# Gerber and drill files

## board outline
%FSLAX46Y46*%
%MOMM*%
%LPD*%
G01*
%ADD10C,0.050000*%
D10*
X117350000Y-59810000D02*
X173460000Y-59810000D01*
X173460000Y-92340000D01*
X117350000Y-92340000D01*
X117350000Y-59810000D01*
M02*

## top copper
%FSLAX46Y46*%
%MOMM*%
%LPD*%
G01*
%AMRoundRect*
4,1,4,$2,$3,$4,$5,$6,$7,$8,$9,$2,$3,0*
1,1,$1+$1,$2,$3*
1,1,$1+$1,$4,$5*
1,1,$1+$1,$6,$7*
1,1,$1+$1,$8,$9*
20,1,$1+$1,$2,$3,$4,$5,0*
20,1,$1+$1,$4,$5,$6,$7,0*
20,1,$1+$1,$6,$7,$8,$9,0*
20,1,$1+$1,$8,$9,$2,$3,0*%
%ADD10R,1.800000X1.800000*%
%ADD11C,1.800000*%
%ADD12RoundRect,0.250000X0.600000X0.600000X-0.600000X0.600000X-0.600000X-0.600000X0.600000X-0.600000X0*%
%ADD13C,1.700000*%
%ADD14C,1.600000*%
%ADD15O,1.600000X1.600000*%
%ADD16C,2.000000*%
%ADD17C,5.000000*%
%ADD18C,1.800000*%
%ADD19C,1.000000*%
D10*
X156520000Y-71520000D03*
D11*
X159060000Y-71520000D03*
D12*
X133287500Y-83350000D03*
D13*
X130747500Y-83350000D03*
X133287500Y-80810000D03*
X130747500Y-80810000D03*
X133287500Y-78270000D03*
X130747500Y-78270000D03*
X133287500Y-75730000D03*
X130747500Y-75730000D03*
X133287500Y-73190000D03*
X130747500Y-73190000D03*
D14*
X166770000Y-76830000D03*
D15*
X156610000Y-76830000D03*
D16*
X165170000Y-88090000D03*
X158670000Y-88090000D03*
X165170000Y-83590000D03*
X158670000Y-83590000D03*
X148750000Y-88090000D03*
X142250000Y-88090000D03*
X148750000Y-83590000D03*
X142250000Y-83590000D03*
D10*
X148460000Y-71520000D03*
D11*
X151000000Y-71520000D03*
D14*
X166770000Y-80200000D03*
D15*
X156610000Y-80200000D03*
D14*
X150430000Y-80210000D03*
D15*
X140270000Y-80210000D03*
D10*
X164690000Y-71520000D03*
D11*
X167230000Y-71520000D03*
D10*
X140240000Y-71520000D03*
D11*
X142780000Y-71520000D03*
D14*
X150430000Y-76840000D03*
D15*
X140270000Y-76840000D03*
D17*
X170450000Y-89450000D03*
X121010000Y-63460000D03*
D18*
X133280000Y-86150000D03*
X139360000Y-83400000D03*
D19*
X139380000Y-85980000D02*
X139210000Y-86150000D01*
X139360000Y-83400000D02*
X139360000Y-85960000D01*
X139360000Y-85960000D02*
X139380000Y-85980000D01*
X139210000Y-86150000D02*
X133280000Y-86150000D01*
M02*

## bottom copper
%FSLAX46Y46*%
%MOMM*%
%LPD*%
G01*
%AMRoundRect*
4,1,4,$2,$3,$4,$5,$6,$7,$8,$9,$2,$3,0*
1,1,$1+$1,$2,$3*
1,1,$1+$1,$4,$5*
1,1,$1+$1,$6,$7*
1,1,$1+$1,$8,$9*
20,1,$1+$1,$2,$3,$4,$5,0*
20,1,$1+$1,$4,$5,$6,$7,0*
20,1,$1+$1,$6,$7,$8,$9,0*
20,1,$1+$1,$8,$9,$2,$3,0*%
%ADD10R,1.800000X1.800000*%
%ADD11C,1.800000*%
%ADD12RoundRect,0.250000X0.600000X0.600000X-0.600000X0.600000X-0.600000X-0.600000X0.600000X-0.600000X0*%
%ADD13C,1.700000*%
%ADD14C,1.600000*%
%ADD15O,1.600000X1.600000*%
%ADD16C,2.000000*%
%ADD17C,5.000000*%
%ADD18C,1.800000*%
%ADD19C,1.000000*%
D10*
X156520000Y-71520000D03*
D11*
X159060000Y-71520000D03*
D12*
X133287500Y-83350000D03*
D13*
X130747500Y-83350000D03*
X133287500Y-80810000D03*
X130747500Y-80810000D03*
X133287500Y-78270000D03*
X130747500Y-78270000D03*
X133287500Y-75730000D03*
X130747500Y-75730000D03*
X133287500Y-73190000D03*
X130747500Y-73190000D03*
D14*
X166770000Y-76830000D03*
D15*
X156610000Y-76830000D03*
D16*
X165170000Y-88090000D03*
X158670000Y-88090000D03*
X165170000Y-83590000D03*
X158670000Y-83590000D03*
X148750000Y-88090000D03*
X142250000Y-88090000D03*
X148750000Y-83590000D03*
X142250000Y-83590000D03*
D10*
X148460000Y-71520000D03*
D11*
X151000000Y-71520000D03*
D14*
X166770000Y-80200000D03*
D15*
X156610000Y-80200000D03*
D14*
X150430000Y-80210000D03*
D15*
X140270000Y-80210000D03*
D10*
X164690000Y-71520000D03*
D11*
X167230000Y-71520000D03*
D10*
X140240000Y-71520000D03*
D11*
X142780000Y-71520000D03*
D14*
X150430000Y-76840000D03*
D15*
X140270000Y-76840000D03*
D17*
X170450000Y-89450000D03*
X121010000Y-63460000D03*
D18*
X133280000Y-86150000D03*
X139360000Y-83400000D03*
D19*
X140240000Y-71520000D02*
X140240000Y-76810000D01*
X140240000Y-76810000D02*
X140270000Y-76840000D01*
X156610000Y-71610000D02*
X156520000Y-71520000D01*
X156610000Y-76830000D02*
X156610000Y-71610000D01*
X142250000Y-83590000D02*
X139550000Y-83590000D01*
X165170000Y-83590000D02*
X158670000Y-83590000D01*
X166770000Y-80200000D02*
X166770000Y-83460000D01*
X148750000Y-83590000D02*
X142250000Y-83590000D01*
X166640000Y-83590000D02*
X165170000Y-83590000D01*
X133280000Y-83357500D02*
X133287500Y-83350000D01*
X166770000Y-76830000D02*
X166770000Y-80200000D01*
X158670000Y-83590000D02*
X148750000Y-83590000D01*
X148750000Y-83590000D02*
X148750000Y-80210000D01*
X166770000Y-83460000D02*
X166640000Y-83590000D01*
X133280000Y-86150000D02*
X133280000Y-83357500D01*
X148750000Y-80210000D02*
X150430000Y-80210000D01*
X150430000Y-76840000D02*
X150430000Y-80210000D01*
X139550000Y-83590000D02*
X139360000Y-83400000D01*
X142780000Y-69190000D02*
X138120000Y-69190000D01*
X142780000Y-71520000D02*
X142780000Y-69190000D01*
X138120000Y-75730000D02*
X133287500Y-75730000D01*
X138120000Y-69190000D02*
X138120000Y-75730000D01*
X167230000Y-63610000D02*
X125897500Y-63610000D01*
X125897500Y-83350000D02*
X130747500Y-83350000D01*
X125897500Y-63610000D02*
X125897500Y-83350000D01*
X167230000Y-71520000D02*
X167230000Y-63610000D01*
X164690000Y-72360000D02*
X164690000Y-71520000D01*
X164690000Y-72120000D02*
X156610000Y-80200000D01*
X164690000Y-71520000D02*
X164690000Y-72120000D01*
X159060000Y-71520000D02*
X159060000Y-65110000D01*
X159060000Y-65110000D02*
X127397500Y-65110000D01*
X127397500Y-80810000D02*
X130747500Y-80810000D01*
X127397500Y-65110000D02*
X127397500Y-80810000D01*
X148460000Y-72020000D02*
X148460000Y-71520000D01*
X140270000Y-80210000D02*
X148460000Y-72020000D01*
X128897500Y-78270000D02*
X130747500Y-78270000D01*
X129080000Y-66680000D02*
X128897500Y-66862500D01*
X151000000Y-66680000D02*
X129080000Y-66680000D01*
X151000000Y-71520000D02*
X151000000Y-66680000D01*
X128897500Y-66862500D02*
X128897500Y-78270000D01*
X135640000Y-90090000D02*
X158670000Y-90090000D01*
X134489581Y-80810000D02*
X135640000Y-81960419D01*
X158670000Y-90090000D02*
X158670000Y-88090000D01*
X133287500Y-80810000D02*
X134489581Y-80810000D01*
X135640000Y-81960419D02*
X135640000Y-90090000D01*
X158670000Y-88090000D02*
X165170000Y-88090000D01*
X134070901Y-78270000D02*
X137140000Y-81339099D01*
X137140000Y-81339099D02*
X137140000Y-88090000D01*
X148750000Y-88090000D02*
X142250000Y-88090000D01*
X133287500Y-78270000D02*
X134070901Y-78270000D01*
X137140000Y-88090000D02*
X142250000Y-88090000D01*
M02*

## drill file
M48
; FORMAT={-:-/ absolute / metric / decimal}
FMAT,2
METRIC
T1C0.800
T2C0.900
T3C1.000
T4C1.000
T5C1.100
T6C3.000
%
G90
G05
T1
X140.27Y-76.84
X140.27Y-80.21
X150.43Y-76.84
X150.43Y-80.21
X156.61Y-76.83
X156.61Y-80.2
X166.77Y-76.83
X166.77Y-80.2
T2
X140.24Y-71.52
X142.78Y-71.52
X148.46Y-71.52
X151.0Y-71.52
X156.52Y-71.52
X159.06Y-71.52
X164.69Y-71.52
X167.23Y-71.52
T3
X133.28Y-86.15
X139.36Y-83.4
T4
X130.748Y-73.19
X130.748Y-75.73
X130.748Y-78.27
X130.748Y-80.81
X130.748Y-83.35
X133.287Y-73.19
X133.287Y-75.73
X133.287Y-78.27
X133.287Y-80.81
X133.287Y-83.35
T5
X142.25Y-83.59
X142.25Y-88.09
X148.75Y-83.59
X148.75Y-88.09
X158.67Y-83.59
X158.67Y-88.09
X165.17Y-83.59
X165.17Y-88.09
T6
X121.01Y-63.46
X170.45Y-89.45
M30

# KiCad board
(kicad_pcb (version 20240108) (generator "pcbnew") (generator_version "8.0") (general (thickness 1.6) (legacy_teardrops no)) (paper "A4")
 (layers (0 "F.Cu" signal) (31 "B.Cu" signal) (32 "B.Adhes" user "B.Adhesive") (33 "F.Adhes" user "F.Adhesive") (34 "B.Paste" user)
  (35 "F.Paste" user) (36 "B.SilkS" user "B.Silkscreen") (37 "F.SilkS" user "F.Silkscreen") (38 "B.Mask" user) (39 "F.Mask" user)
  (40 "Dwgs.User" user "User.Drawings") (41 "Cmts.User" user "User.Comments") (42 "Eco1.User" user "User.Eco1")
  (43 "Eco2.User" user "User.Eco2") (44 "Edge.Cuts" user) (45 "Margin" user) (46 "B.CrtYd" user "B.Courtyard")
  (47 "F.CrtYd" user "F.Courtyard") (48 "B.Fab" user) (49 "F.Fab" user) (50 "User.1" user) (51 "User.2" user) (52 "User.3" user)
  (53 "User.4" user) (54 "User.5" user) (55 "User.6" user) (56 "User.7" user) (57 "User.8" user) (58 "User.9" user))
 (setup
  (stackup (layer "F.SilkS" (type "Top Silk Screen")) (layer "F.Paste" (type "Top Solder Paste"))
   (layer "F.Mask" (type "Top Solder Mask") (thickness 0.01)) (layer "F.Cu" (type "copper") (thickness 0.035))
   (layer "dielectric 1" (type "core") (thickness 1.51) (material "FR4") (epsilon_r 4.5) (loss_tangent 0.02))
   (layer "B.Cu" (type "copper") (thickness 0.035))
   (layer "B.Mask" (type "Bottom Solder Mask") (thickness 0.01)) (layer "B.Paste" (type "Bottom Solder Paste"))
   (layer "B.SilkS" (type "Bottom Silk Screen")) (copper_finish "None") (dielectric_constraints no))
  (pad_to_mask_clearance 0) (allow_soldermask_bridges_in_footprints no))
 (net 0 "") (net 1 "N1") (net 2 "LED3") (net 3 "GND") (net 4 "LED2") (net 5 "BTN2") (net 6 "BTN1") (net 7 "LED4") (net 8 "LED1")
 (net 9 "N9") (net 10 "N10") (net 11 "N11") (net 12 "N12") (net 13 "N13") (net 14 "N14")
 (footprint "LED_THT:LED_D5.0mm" (layer "F.Cu") (at 156.52 71.52)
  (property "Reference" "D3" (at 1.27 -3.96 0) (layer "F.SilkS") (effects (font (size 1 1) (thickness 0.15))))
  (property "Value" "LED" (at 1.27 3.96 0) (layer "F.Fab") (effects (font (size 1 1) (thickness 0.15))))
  (pad "1" thru_hole rect (at 0 0) (size 1.8 1.8) (drill 0.9) (layers "*.Cu" "*.Mask") (remove_unused_layers no) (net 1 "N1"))
  (pad "2" thru_hole circle (at 2.54 0) (size 1.8 1.8) (drill 0.9) (layers "*.Cu" "*.Mask") (remove_unused_layers no) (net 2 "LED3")))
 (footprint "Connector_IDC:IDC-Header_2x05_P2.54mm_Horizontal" (layer "F.Cu") (at 133.2875 83.35 180)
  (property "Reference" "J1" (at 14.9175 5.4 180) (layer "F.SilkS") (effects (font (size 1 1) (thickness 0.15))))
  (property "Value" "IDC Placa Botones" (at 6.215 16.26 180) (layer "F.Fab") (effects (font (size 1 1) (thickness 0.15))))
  (pad "1" thru_hole roundrect (at 0 0 180) (size 1.7 1.7) (drill 1) (layers "*.Cu" "*.Mask") (remove_unused_layers no)
   (roundrect_rratio 0.147059) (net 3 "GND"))
  (pad "2" thru_hole circle (at 2.54 0 180) (size 1.7 1.7) (drill 1) (layers "*.Cu" "*.Mask") (remove_unused_layers no) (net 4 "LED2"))
  (pad "3" thru_hole circle (at 0 2.54 180) (size 1.7 1.7) (drill 1) (layers "*.Cu" "*.Mask") (remove_unused_layers no) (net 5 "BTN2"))
  (pad "4" thru_hole circle (at 2.54 2.54 180) (size 1.7 1.7) (drill 1) (layers "*.Cu" "*.Mask") (remove_unused_layers no) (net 2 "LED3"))
  (pad "5" thru_hole circle (at 0 5.08 180) (size 1.7 1.7) (drill 1) (layers "*.Cu" "*.Mask") (remove_unused_layers no) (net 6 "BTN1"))
  (pad "6" thru_hole circle (at 2.54 5.08 180) (size 1.7 1.7) (drill 1) (layers "*.Cu" "*.Mask") (remove_unused_layers no) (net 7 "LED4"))
  (pad "7" thru_hole circle (at 0 7.62 180) (size 1.7 1.7) (drill 1) (layers "*.Cu" "*.Mask") (remove_unused_layers no) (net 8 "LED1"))
  (pad "8" thru_hole circle (at 2.54 7.62 180) (size 1.7 1.7) (drill 1) (layers "*.Cu" "*.Mask") (remove_unused_layers no) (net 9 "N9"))
  (pad "9" thru_hole circle (at 0 10.16 180) (size 1.7 1.7) (drill 1) (layers "*.Cu" "*.Mask") (remove_unused_layers no) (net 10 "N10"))
  (pad "10" thru_hole circle (at 2.54 10.16 180) (size 1.7 1.7) (drill 1) (layers "*.Cu" "*.Mask") (remove_unused_layers no) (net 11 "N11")))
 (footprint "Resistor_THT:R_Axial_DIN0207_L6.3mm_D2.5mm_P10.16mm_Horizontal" (layer "F.Cu") (at 166.77 76.83 180)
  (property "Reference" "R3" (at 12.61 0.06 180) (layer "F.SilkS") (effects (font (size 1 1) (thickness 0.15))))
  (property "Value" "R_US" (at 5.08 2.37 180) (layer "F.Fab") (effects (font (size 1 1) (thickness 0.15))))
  (pad "1" thru_hole circle (at 0 0 180) (size 1.6 1.6) (drill 0.8) (layers "*.Cu" "*.Mask") (remove_unused_layers no) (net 3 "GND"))
  (pad "2" thru_hole oval (at 10.16 0 180) (size 1.6 1.6) (drill 0.8) (layers "*.Cu" "*.Mask") (remove_unused_layers no) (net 1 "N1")))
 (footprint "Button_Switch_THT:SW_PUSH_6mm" (layer "F.Cu") (at 165.17 88.09 180)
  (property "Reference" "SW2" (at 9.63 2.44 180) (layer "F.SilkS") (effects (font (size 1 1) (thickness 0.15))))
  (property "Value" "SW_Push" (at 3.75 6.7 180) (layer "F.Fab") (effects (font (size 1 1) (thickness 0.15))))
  (pad "1" thru_hole circle (at 0 0 270) (size 2 2) (drill 1.1) (layers "*.Cu" "*.Mask") (remove_unused_layers no) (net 5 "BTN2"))
  (pad "1" thru_hole circle (at 6.5 0 270) (size 2 2) (drill 1.1) (layers "*.Cu" "*.Mask") (remove_unused_layers no) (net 5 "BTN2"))
  (pad "2" thru_hole circle (at 0 4.5 270) (size 2 2) (drill 1.1) (layers "*.Cu" "*.Mask") (remove_unused_layers no) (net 3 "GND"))
  (pad "2" thru_hole circle (at 6.5 4.5 270) (size 2 2) (drill 1.1) (layers "*.Cu" "*.Mask") (remove_unused_layers no) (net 3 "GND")))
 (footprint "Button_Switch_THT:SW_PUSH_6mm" (layer "F.Cu") (at 148.75 88.09 180)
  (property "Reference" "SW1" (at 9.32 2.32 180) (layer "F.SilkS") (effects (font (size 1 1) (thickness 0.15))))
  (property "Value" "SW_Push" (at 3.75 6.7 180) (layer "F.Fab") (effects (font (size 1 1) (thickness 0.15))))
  (pad "1" thru_hole circle (at 0 0 270) (size 2 2) (drill 1.1) (layers "*.Cu" "*.Mask") (remove_unused_layers no) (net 6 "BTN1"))
  (pad "1" thru_hole circle (at 6.5 0 270) (size 2 2) (drill 1.1) (layers "*.Cu" "*.Mask") (remove_unused_layers no) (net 6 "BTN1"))
  (pad "2" thru_hole circle (at 0 4.5 270) (size 2 2) (drill 1.1) (layers "*.Cu" "*.Mask") (remove_unused_layers no) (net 3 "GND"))
  (pad "2" thru_hole circle (at 6.5 4.5 270) (size 2 2) (drill 1.1) (layers "*.Cu" "*.Mask") (remove_unused_layers no) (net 3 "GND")))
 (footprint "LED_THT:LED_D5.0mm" (layer "F.Cu") (at 148.46 71.52)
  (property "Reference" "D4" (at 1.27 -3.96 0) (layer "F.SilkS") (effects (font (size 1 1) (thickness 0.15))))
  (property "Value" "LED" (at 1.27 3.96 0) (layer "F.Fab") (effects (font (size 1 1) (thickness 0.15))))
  (pad "1" thru_hole rect (at 0 0) (size 1.8 1.8) (drill 0.9) (layers "*.Cu" "*.Mask") (remove_unused_layers no) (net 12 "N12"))
  (pad "2" thru_hole circle (at 2.54 0) (size 1.8 1.8) (drill 0.9) (layers "*.Cu" "*.Mask") (remove_unused_layers no) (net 7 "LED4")))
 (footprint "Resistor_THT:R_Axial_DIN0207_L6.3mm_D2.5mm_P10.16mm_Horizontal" (layer "F.Cu") (at 166.77 80.2 180)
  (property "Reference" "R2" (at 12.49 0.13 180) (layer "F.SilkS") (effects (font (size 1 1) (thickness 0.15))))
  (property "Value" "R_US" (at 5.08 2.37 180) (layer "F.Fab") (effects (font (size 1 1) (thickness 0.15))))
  (pad "1" thru_hole circle (at 0 0 180) (size 1.6 1.6) (drill 0.8) (layers "*.Cu" "*.Mask") (remove_unused_layers no) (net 3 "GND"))
  (pad "2" thru_hole oval (at 10.16 0 180) (size 1.6 1.6) (drill 0.8) (layers "*.Cu" "*.Mask") (remove_unused_layers no) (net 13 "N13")))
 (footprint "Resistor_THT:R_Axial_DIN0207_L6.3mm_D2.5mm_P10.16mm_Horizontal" (layer "F.Cu") (at 150.43 80.21 180)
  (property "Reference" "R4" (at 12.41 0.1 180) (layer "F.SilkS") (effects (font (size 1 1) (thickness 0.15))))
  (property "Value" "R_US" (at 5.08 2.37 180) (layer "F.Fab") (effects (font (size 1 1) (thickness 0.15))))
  (pad "1" thru_hole circle (at 0 0 180) (size 1.6 1.6) (drill 0.8) (layers "*.Cu" "*.Mask") (remove_unused_layers no) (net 3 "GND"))
  (pad "2" thru_hole oval (at 10.16 0 180) (size 1.6 1.6) (drill 0.8) (layers "*.Cu" "*.Mask") (remove_unused_layers no) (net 12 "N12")))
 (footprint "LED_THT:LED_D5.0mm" (layer "F.Cu") (at 164.69 71.52)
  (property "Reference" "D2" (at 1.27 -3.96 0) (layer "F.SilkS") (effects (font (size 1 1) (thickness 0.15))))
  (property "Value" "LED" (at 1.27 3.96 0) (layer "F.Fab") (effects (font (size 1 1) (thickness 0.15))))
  (pad "1" thru_hole rect (at 0 0) (size 1.8 1.8) (drill 0.9) (layers "*.Cu" "*.Mask") (remove_unused_layers no) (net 13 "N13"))
  (pad "2" thru_hole circle (at 2.54 0) (size 1.8 1.8) (drill 0.9) (layers "*.Cu" "*.Mask") (remove_unused_layers no) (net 4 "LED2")))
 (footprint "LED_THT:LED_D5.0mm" (layer "F.Cu") (at 140.24 71.52)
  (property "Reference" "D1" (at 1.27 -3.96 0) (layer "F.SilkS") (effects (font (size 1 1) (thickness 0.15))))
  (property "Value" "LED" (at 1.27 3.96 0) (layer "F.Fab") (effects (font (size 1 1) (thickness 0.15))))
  (pad "1" thru_hole rect (at 0 0) (size 1.8 1.8) (drill 0.9) (layers "*.Cu" "*.Mask") (remove_unused_layers no) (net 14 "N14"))
  (pad "2" thru_hole circle (at 2.54 0) (size 1.8 1.8) (drill 0.9) (layers "*.Cu" "*.Mask") (remove_unused_layers no) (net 8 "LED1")))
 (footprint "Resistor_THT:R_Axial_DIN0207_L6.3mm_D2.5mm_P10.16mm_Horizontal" (layer "F.Cu") (at 150.43 76.84 180)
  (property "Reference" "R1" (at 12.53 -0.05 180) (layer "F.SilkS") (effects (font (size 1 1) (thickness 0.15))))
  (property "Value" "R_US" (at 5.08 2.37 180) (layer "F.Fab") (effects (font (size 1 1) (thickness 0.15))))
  (pad "1" thru_hole circle (at 0 0 180) (size 1.6 1.6) (drill 0.8) (layers "*.Cu" "*.Mask") (remove_unused_layers no) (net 3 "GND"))
  (pad "2" thru_hole oval (at 10.16 0 180) (size 1.6 1.6) (drill 0.8) (layers "*.Cu" "*.Mask") (remove_unused_layers no) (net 14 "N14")))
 (gr_rect (start 117.35 59.81) (end 173.46 92.34) (stroke (width 0.05) (type default)) (fill none) (layer "Edge.Cuts"))
 (via (at 170.45 89.45) (size 5) (drill 3) (layers "F.Cu" "B.Cu") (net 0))
 (via (at 121.01 63.46) (size 5) (drill 3) (layers "F.Cu" "B.Cu") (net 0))
 (segment (start 140.24 71.52) (end 140.24 76.81) (width 1) (layer "B.Cu") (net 14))
 (segment (start 140.24 76.81) (end 140.27 76.84) (width 1) (layer "B.Cu") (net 14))
 (segment (start 156.61 71.61) (end 156.52 71.52) (width 1) (layer "B.Cu") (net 1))
 (segment (start 156.61 76.83) (end 156.61 71.61) (width 1) (layer "B.Cu") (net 1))
 (segment (start 139.38 85.98) (end 139.21 86.15) (width 1) (layer "F.Cu") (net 3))
 (segment (start 139.36 83.4) (end 139.36 85.96) (width 1) (layer "F.Cu") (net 3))
 (segment (start 139.36 85.96) (end 139.38 85.98) (width 1) (layer "F.Cu") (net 3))
 (segment (start 139.21 86.15) (end 133.28 86.15) (width 1) (layer "F.Cu") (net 3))
 (via (at 133.28 86.15) (size 1.8) (drill 1) (layers "F.Cu" "B.Cu") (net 3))
 (via (at 139.36 83.4) (size 1.8) (drill 1) (layers "F.Cu" "B.Cu") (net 3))
 (segment (start 142.25 83.59) (end 139.55 83.59) (width 1) (layer "B.Cu") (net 3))
 (segment (start 165.17 83.59) (end 158.67 83.59) (width 1) (layer "B.Cu") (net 3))
 (segment (start 166.77 80.2) (end 166.77 83.46) (width 1) (layer "B.Cu") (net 3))
 (segment (start 148.75 83.59) (end 142.25 83.59) (width 1) (layer "B.Cu") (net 3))
 (segment (start 166.64 83.59) (end 165.17 83.59) (width 1) (layer "B.Cu") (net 3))
 (segment (start 133.28 83.3575) (end 133.2875 83.35) (width 1) (layer "B.Cu") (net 3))
 (segment (start 166.77 76.83) (end 166.77 80.2) (width 1) (layer "B.Cu") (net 3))
 (segment (start 158.67 83.59) (end 148.75 83.59) (width 1) (layer "B.Cu") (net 3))
 (segment (start 148.75 83.59) (end 148.75 80.21) (width 1) (layer "B.Cu") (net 3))
 (segment (start 166.77 83.46) (end 166.64 83.59) (width 1) (layer "B.Cu") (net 3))
 (segment (start 133.28 86.15) (end 133.28 83.3575) (width 1) (layer "B.Cu") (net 3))
 (segment (start 148.75 80.21) (end 150.43 80.21) (width 1) (layer "B.Cu") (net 3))
 (segment (start 150.43 76.84) (end 150.43 80.21) (width 1) (layer "B.Cu") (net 3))
 (segment (start 139.55 83.59) (end 139.36 83.4) (width 1) (layer "B.Cu") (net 3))
 (segment (start 142.78 69.19) (end 138.12 69.19) (width 1) (layer "B.Cu") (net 8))
 (segment (start 142.78 71.52) (end 142.78 69.19) (width 1) (layer "B.Cu") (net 8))
 (segment (start 138.12 75.73) (end 133.2875 75.73) (width 1) (layer "B.Cu") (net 8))
 (segment (start 138.12 69.19) (end 138.12 75.73) (width 1) (layer "B.Cu") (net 8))
 (segment (start 167.23 63.61) (end 125.8975 63.61) (width 1) (layer "B.Cu") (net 4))
 (segment (start 125.8975 83.35) (end 130.7475 83.35) (width 1) (layer "B.Cu") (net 4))
 (segment (start 125.8975 63.61) (end 125.8975 83.35) (width 1) (layer "B.Cu") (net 4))
 (segment (start 167.23 71.52) (end 167.23 63.61) (width 1) (layer "B.Cu") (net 4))
 (segment (start 164.69 72.36) (end 164.69 71.52) (width 1) (layer "B.Cu") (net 13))
 (segment (start 164.69 72.12) (end 156.61 80.2) (width 1) (layer "B.Cu") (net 13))
 (segment (start 164.69 71.52) (end 164.69 72.12) (width 1) (layer "B.Cu") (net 13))
 (segment (start 159.06 71.52) (end 159.06 65.11) (width 1) (layer "B.Cu") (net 2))
 (segment (start 159.06 65.11) (end 127.3975 65.11) (width 1) (layer "B.Cu") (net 2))
 (segment (start 127.3975 80.81) (end 130.7475 80.81) (width 1) (layer "B.Cu") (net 2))
 (segment (start 127.3975 65.11) (end 127.3975 80.81) (width 1) (layer "B.Cu") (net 2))
 (segment (start 148.46 72.02) (end 148.46 71.52) (width 1) (layer "B.Cu") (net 12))
 (segment (start 140.27 80.21) (end 148.46 72.02) (width 1) (layer "B.Cu") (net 12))
 (segment (start 128.8975 78.27) (end 130.7475 78.27) (width 1) (layer "B.Cu") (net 7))
 (segment (start 129.08 66.68) (end 128.8975 66.8625) (width 1) (layer "B.Cu") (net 7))
 (segment (start 151 66.68) (end 129.08 66.68) (width 1) (layer "B.Cu") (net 7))
 (segment (start 151 71.52) (end 151 66.68) (width 1) (layer "B.Cu") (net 7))
 (segment (start 128.8975 66.8625) (end 128.8975 78.27) (width 1) (layer "B.Cu") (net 7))
 (segment (start 135.64 90.09) (end 158.67 90.09) (width 1) (layer "B.Cu") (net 5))
 (segment (start 134.489581 80.81) (end 135.64 81.960419) (width 1) (layer "B.Cu") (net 5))
 (segment (start 158.67 90.09) (end 158.67 88.09) (width 1) (layer "B.Cu") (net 5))
 (segment (start 133.2875 80.81) (end 134.489581 80.81) (width 1) (layer "B.Cu") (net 5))
 (segment (start 135.64 81.960419) (end 135.64 90.09) (width 1) (layer "B.Cu") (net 5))
 (segment (start 158.67 88.09) (end 165.17 88.09) (width 1) (layer "B.Cu") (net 5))
 (segment (start 134.070901 78.27) (end 137.14 81.339099) (width 1) (layer "B.Cu") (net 6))
 (segment (start 137.14 81.339099) (end 137.14 88.09) (width 1) (layer "B.Cu") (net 6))
 (segment (start 148.75 88.09) (end 142.25 88.09) (width 1) (layer "B.Cu") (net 6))
 (segment (start 133.2875 78.27) (end 134.070901 78.27) (width 1) (layer "B.Cu") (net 6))
 (segment (start 137.14 88.09) (end 142.25 88.09) (width 1) (layer "B.Cu") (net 6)))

